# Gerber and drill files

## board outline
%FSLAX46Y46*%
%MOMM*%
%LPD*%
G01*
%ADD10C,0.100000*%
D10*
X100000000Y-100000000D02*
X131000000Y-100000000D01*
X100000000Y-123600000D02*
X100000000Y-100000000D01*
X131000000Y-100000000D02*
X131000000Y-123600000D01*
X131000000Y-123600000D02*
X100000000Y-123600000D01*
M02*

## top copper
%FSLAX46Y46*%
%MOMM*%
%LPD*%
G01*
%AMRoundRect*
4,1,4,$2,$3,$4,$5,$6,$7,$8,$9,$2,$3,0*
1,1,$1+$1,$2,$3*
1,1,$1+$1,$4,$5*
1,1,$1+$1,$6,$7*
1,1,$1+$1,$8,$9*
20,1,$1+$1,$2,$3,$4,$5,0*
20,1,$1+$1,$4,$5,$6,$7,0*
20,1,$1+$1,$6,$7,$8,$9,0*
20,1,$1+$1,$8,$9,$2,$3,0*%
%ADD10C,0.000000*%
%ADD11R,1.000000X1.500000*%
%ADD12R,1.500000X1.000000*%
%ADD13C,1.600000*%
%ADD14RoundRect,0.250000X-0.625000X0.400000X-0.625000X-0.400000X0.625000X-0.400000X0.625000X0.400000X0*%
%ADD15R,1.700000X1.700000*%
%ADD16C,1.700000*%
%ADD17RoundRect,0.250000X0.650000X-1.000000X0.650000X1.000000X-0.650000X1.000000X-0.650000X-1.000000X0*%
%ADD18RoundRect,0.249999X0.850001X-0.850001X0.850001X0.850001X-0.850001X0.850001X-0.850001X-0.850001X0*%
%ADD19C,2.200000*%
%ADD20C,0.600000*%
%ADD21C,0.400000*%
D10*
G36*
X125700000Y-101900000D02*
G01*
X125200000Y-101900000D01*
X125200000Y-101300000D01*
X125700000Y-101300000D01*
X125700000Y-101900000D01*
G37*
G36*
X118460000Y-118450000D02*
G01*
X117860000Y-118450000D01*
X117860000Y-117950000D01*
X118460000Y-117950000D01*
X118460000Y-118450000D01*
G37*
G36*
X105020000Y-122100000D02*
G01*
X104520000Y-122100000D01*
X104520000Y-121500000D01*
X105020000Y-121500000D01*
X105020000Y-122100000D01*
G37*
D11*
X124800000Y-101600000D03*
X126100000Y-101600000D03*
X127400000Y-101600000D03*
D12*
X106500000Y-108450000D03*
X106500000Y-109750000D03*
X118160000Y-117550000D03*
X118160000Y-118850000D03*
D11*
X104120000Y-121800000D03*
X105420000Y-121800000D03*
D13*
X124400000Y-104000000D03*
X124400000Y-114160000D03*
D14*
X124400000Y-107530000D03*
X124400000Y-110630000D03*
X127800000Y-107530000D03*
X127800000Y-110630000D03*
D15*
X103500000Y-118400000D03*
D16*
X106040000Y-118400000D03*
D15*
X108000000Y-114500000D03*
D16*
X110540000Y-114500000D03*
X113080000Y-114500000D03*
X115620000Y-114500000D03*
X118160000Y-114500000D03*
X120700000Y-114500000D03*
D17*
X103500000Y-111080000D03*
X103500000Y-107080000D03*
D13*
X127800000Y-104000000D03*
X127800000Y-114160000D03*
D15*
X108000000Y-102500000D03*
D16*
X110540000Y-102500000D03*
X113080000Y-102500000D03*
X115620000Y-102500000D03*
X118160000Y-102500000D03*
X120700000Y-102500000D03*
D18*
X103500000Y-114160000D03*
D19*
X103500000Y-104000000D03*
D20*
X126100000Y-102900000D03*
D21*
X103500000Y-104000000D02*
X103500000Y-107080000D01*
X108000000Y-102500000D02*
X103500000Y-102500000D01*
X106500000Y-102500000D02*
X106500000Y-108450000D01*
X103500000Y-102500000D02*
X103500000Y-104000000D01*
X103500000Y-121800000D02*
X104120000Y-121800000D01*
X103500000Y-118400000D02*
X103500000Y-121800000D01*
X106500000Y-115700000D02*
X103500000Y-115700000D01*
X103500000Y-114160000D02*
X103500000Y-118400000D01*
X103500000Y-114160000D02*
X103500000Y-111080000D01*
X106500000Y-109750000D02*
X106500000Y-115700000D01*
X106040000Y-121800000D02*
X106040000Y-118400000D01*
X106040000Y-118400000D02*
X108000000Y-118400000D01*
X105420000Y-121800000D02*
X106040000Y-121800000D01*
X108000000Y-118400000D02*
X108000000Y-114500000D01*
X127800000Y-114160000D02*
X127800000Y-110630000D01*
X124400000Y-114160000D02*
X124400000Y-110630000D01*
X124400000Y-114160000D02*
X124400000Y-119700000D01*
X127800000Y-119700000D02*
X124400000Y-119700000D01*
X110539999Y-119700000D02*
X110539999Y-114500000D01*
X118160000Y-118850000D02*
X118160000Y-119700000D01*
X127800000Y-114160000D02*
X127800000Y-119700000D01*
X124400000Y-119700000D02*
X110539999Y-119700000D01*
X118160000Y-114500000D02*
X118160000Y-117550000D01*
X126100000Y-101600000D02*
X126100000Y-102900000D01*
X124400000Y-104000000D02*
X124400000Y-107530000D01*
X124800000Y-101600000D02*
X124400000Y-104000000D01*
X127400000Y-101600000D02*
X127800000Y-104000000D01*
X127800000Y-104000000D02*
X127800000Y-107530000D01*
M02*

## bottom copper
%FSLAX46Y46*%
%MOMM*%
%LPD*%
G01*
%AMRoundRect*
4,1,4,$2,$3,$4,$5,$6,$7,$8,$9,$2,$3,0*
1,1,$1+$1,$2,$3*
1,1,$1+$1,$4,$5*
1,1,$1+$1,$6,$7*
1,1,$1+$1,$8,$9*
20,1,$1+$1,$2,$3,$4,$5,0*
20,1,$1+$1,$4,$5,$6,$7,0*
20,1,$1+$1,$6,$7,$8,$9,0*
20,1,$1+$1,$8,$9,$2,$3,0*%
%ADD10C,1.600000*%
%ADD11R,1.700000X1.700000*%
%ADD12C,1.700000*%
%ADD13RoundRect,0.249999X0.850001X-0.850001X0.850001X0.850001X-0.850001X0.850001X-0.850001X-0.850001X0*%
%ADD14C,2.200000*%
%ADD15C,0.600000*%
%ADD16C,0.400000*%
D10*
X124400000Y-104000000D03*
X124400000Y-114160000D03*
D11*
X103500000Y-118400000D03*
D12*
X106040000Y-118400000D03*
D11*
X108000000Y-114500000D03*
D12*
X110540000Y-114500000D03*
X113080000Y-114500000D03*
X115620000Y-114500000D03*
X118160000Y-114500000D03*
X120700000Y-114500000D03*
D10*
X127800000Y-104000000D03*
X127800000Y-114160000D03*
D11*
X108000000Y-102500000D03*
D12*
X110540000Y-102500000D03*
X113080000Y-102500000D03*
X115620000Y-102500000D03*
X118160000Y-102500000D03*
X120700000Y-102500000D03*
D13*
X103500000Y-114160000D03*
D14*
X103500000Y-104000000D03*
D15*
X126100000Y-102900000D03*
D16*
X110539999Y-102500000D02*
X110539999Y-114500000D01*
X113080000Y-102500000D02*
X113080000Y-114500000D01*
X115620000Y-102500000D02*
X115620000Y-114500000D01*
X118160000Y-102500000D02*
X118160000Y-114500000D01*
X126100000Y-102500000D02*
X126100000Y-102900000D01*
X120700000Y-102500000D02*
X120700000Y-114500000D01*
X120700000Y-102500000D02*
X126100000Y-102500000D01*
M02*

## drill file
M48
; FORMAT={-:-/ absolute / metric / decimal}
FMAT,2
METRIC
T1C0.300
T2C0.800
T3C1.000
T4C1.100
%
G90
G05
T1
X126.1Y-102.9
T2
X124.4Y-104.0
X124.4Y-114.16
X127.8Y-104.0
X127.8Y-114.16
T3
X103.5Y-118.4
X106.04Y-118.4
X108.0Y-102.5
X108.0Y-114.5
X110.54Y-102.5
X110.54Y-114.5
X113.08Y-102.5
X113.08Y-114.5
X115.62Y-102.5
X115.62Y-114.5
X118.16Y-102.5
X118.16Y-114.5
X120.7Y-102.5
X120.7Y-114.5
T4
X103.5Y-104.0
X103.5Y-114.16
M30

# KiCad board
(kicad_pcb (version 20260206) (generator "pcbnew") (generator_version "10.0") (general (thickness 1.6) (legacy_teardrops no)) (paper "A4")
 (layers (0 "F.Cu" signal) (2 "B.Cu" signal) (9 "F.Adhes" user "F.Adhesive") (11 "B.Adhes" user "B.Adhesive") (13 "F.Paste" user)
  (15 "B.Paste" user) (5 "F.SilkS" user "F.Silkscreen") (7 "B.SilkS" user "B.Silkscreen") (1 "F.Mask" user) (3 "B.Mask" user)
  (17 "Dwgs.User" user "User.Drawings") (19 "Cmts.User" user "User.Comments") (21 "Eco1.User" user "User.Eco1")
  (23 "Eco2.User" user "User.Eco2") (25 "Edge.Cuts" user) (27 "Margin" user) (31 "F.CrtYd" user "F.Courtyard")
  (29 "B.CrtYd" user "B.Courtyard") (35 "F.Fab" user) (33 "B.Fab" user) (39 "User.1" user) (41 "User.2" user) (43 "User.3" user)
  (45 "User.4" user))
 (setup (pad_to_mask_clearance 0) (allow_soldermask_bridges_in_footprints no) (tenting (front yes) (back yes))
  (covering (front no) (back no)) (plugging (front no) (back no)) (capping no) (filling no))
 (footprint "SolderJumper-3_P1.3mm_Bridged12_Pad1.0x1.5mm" (layer "F.Cu") (at 126.1 101.6)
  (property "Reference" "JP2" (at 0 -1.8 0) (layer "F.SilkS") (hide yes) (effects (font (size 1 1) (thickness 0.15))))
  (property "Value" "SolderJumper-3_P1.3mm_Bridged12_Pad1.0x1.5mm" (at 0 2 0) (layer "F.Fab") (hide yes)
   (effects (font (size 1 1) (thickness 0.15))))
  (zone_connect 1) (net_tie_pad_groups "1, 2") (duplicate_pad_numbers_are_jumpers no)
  (fp_poly (pts (xy -0.9 -0.3) (xy -0.4 -0.3) (xy -0.4 0.3) (xy -0.9 0.3)) (stroke (width 0) (type solid)) (fill yes) (layer "F.Cu"))
  (pad "1" smd rect (at -1.3 0) (size 1 1.5) (layers "F.Cu" "F.Mask") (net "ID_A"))
  (pad "2" smd rect (at 0 0) (size 1 1.5) (layers "F.Cu" "F.Mask") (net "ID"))
  (pad "3" smd rect (at 1.3 0) (size 1 1.5) (layers "F.Cu" "F.Mask") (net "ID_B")))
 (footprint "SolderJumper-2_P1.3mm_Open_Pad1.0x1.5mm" (layer "F.Cu") (at 106.5 109.1 -90)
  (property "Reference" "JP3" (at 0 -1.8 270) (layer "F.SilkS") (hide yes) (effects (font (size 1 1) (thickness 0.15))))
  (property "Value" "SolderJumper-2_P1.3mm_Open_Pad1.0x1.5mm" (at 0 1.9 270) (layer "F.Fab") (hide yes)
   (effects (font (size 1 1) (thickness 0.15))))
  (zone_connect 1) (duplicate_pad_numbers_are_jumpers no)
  (pad "1" smd rect (at -0.65 0 270) (size 1 1.5) (layers "F.Cu" "F.Mask") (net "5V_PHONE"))
  (pad "2" smd rect (at 0.65 0 270) (size 1 1.5) (layers "F.Cu" "F.Mask") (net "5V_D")))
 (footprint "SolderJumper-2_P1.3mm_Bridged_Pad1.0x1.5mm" (layer "F.Cu") (at 118.16 118.2 -90)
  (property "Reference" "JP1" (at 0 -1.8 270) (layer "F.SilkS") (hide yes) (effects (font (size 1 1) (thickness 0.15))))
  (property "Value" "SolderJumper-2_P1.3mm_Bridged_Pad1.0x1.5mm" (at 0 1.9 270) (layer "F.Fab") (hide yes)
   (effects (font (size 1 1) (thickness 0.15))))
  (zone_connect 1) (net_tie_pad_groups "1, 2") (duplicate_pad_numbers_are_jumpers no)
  (fp_poly (pts (xy -0.25 -0.3) (xy 0.25 -0.3) (xy 0.25 0.3) (xy -0.25 0.3)) (stroke (width 0) (type solid)) (fill yes) (layer "F.Cu"))
  (pad "1" smd rect (at -0.65 0 270) (size 1 1.5) (layers "F.Cu" "F.Mask") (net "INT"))
  (pad "2" smd rect (at 0.65 0 270) (size 1 1.5) (layers "F.Cu" "F.Mask") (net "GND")))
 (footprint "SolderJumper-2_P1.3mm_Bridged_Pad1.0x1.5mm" (layer "F.Cu") (at 104.77 121.8)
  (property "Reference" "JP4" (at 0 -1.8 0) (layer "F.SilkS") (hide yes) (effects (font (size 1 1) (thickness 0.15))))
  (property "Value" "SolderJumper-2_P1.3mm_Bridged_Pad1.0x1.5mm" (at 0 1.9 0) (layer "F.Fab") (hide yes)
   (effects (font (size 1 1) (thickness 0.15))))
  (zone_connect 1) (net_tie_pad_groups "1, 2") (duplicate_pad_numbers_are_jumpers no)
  (fp_poly (pts (xy -0.25 -0.3) (xy 0.25 -0.3) (xy 0.25 0.3) (xy -0.25 0.3)) (stroke (width 0) (type solid)) (fill yes) (layer "F.Cu"))
  (pad "1" smd rect (at -0.65 0) (size 1 1.5) (layers "F.Cu" "F.Mask") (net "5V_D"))
  (pad "2" smd rect (at 0.65 0) (size 1 1.5) (layers "F.Cu" "F.Mask") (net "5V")))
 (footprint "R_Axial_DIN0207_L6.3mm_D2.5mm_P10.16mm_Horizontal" (layer "F.Cu") (at 124.4 104 -90)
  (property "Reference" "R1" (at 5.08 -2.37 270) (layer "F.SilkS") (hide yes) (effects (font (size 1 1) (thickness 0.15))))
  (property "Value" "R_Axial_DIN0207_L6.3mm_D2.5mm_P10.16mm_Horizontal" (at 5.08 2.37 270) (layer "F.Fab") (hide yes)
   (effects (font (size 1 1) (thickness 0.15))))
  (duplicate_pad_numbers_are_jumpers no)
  (pad "1" thru_hole circle (at 0 0 270) (size 1.6 1.6) (drill 0.8) (layers "*.Cu" "*.Mask") (remove_unused_layers no) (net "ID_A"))
  (pad "2" thru_hole circle (at 10.16 0 270) (size 1.6 1.6) (drill 0.8) (layers "*.Cu" "*.Mask") (remove_unused_layers no) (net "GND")))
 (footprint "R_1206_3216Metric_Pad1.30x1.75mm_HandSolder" (layer "F.Cu") (at 124.4 109.08 -90)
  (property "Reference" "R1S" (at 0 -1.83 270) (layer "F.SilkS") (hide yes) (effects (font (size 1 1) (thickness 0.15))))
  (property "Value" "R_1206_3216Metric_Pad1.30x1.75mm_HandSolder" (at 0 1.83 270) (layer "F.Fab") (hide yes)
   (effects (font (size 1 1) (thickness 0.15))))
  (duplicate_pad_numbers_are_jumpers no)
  (pad "1" smd roundrect (at -1.55 0 270) (size 1.3 1.75) (layers "F.Cu" "F.Mask" "F.Paste") (roundrect_rratio 0.192308) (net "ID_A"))
  (pad "2" smd roundrect (at 1.55 0 270) (size 1.3 1.75) (layers "F.Cu" "F.Mask" "F.Paste") (roundrect_rratio 0.192308) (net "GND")))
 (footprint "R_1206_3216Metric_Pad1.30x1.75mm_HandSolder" (layer "F.Cu") (at 127.8 109.08 -90)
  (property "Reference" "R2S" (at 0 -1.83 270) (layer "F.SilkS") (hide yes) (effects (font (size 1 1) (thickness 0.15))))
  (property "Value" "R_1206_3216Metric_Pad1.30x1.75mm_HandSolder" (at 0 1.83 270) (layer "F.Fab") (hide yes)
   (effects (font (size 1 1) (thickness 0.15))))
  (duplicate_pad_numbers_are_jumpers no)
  (pad "1" smd roundrect (at -1.55 0 270) (size 1.3 1.75) (layers "F.Cu" "F.Mask" "F.Paste") (roundrect_rratio 0.192308) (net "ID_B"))
  (pad "2" smd roundrect (at 1.55 0 270) (size 1.3 1.75) (layers "F.Cu" "F.Mask" "F.Paste") (roundrect_rratio 0.192308) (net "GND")))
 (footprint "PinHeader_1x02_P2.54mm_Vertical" (layer "F.Cu") (at 103.5 118.4 90)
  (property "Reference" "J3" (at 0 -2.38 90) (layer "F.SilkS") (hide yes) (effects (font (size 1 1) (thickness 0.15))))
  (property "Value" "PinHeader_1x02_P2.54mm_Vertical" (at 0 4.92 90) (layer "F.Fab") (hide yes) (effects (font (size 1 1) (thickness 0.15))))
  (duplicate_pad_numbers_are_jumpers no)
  (pad "1" thru_hole rect (at 0 0 90) (size 1.7 1.7) (drill 1) (layers "*.Cu" "*.Mask") (remove_unused_layers no) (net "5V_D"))
  (pad "2" thru_hole circle (at 0 2.54 90) (size 1.7 1.7) (drill 1) (layers "*.Cu" "*.Mask") (remove_unused_layers no) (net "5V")))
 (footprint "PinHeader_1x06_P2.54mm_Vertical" (layer "F.Cu") (at 108 114.5 90)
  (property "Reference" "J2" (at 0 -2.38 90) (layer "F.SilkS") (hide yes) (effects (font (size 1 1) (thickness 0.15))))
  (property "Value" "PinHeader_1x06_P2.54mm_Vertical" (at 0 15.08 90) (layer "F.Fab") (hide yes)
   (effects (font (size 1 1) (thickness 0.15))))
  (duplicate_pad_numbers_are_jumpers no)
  (pad "1" thru_hole rect (at 0 0 90) (size 1.7 1.7) (drill 1) (layers "*.Cu" "*.Mask") (remove_unused_layers no) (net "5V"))
  (pad "2" thru_hole circle (at 0 2.54 90) (size 1.7 1.7) (drill 1) (layers "*.Cu" "*.Mask") (remove_unused_layers no) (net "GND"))
  (pad "3" thru_hole circle (at 0 5.08 90) (size 1.7 1.7) (drill 1) (layers "*.Cu" "*.Mask") (remove_unused_layers no) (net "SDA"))
  (pad "4" thru_hole circle (at 0 7.62 90) (size 1.7 1.7) (drill 1) (layers "*.Cu" "*.Mask") (remove_unused_layers no) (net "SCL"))
  (pad "5" thru_hole circle (at 0 10.16 90) (size 1.7 1.7) (drill 1) (layers "*.Cu" "*.Mask") (remove_unused_layers no) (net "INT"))
  (pad "6" thru_hole circle (at 0 12.7 90) (size 1.7 1.7) (drill 1) (layers "*.Cu" "*.Mask") (remove_unused_layers no) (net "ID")))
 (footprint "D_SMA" (layer "F.Cu") (at 103.5 109.08 90)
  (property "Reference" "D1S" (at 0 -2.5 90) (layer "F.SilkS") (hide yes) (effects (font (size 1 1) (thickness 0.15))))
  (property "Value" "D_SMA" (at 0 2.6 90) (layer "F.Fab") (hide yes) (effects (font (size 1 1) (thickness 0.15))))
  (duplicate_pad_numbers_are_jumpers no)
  (pad "1" smd roundrect (at -2 0 90) (size 2.5 1.8) (layers "F.Cu" "F.Mask" "F.Paste") (roundrect_rratio 0.1388888889) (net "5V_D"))
  (pad "2" smd roundrect (at 2 0 90) (size 2.5 1.8) (layers "F.Cu" "F.Mask" "F.Paste") (roundrect_rratio 0.1388888889) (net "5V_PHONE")))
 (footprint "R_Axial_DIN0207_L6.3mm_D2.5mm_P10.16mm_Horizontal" (layer "F.Cu") (at 127.8 104 -90)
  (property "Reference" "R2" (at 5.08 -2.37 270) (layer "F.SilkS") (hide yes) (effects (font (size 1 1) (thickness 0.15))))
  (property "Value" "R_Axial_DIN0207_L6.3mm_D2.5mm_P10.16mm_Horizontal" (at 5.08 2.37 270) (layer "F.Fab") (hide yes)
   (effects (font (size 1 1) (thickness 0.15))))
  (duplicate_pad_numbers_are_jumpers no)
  (pad "1" thru_hole circle (at 0 0 270) (size 1.6 1.6) (drill 0.8) (layers "*.Cu" "*.Mask") (remove_unused_layers no) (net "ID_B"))
  (pad "2" thru_hole circle (at 10.16 0 270) (size 1.6 1.6) (drill 0.8) (layers "*.Cu" "*.Mask") (remove_unused_layers no) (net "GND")))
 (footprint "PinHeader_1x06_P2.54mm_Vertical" (layer "F.Cu") (at 108 102.5 90)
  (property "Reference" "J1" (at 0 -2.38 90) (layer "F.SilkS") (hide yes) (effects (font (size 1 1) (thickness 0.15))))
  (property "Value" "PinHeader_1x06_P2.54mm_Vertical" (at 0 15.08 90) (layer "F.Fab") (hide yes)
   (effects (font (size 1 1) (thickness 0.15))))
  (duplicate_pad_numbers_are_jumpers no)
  (pad "1" thru_hole rect (at 0 0 90) (size 1.7 1.7) (drill 1) (layers "*.Cu" "*.Mask") (remove_unused_layers no) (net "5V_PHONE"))
  (pad "2" thru_hole circle (at 0 2.54 90) (size 1.7 1.7) (drill 1) (layers "*.Cu" "*.Mask") (remove_unused_layers no) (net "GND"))
  (pad "3" thru_hole circle (at 0 5.08 90) (size 1.7 1.7) (drill 1) (layers "*.Cu" "*.Mask") (remove_unused_layers no) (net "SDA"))
  (pad "4" thru_hole circle (at 0 7.62 90) (size 1.7 1.7) (drill 1) (layers "*.Cu" "*.Mask") (remove_unused_layers no) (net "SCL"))
  (pad "5" thru_hole circle (at 0 10.16 90) (size 1.7 1.7) (drill 1) (layers "*.Cu" "*.Mask") (remove_unused_layers no) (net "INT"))
  (pad "6" thru_hole circle (at 0 12.7 90) (size 1.7 1.7) (drill 1) (layers "*.Cu" "*.Mask") (remove_unused_layers no) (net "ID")))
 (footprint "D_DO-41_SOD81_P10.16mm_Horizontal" (layer "F.Cu") (at 103.5 114.16 90)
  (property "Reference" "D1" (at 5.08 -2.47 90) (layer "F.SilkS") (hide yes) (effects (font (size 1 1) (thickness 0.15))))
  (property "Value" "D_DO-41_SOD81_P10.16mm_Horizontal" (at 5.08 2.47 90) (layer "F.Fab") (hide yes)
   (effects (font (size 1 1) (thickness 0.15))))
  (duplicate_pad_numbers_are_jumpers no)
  (pad "1" thru_hole roundrect (at 0 0 90) (size 2.2 2.2) (drill 1.1) (layers "*.Cu" "*.Mask") (remove_unused_layers no)
   (roundrect_rratio 0.113636) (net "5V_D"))
  (pad "2" thru_hole circle (at 10.16 0 90) (size 2.2 2.2) (drill 1.1) (layers "*.Cu" "*.Mask") (remove_unused_layers no) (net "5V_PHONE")))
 (gr_line (start 100 100) (end 131 100) (stroke (width 0.1) (type default)) (layer "Edge.Cuts"))
 (gr_line (start 100 123.6) (end 100 100) (stroke (width 0.1) (type default)) (layer "Edge.Cuts"))
 (gr_line (start 131 100) (end 131 123.6) (stroke (width 0.1) (type default)) (layer "Edge.Cuts"))
 (gr_line (start 131 123.6) (end 100 123.6) (stroke (width 0.1) (type default)) (layer "Edge.Cuts"))
 (segment (start 103.5 104) (end 103.5 107.08) (width 0.4) (layer "F.Cu") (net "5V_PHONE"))
 (segment (start 108 102.5) (end 103.5 102.5) (width 0.4) (layer "F.Cu") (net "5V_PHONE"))
 (segment (start 106.5 102.5) (end 106.5 108.45) (width 0.4) (layer "F.Cu") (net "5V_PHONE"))
 (segment (start 103.5 102.5) (end 103.5 104) (width 0.4) (layer "F.Cu") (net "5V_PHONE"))
 (segment (start 103.5 121.8) (end 104.12 121.8) (width 0.4) (layer "F.Cu") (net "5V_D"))
 (segment (start 103.5 118.4) (end 103.5 121.8) (width 0.4) (layer "F.Cu") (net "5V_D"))
 (segment (start 106.5 115.7) (end 103.5 115.7) (width 0.4) (layer "F.Cu") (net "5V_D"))
 (segment (start 103.5 114.16) (end 103.5 118.4) (width 0.4) (layer "F.Cu") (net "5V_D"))
 (segment (start 103.5 114.16) (end 103.5 111.08) (width 0.4) (layer "F.Cu") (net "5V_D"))
 (segment (start 106.5 109.75) (end 106.5 115.7) (width 0.4) (layer "F.Cu") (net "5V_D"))
 (segment (start 106.04 121.8) (end 106.04 118.4) (width 0.4) (layer "F.Cu") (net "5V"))
 (segment (start 106.04 118.4) (end 108 118.4) (width 0.4) (layer "F.Cu") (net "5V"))
 (segment (start 105.42 121.8) (end 106.04 121.8) (width 0.4) (layer "F.Cu") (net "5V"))
 (segment (start 108 118.4) (end 108 114.5) (width 0.4) (layer "F.Cu") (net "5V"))
 (segment (start 127.8 114.16) (end 127.8 110.63) (width 0.4) (layer "F.Cu") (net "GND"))
 (segment (start 124.4 114.16) (end 124.4 110.63) (width 0.4) (layer "F.Cu") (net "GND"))
 (segment (start 124.4 114.16) (end 124.4 119.7) (width 0.4) (layer "F.Cu") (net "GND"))
 (segment (start 127.8 119.7) (end 124.4 119.7) (width 0.4) (layer "F.Cu") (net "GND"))
 (segment (start 110.539999 119.7) (end 110.539999 114.5) (width 0.4) (layer "F.Cu") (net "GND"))
 (segment (start 118.16 118.85) (end 118.16 119.7) (width 0.4) (layer "F.Cu") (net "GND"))
 (segment (start 127.8 114.16) (end 127.8 119.7) (width 0.4) (layer "F.Cu") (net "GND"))
 (segment (start 124.4 119.7) (end 110.539999 119.7) (width 0.4) (layer "F.Cu") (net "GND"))
 (segment (start 110.539999 102.5) (end 110.539999 114.5) (width 0.4) (layer "B.Cu") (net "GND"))
 (segment (start 113.08 102.5) (end 113.08 114.5) (width 0.4) (layer "B.Cu") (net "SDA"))
 (segment (start 115.62 102.5) (end 115.62 114.5) (width 0.4) (layer "B.Cu") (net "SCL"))
 (segment (start 118.16 114.5) (end 118.16 117.55) (width 0.4) (layer "F.Cu") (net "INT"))
 (segment (start 118.16 102.5) (end 118.16 114.5) (width 0.4) (layer "B.Cu") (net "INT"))
 (segment (start 126.1 101.6) (end 126.1 102.9) (width 0.4) (layer "F.Cu") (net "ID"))
 (via (at 126.1 102.9) (size 0.6) (drill 0.3) (layers "F.Cu" "B.Cu") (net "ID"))
 (segment (start 126.1 102.5) (end 126.1 102.9) (width 0.4) (layer "B.Cu") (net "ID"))
 (segment (start 120.7 102.5) (end 120.7 114.5) (width 0.4) (layer "B.Cu") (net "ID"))
 (segment (start 120.7 102.5) (end 126.1 102.5) (width 0.4) (layer "B.Cu") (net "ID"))
 (segment (start 124.4 104) (end 124.4 107.53) (width 0.4) (layer "F.Cu") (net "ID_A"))
 (segment (start 124.8 101.6) (end 124.4 104) (width 0.4) (layer "F.Cu") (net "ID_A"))
 (segment (start 127.4 101.6) (end 127.8 104) (width 0.4) (layer "F.Cu") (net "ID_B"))
 (segment (start 127.8 104) (end 127.8 107.53) (width 0.4) (layer "F.Cu") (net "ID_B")))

